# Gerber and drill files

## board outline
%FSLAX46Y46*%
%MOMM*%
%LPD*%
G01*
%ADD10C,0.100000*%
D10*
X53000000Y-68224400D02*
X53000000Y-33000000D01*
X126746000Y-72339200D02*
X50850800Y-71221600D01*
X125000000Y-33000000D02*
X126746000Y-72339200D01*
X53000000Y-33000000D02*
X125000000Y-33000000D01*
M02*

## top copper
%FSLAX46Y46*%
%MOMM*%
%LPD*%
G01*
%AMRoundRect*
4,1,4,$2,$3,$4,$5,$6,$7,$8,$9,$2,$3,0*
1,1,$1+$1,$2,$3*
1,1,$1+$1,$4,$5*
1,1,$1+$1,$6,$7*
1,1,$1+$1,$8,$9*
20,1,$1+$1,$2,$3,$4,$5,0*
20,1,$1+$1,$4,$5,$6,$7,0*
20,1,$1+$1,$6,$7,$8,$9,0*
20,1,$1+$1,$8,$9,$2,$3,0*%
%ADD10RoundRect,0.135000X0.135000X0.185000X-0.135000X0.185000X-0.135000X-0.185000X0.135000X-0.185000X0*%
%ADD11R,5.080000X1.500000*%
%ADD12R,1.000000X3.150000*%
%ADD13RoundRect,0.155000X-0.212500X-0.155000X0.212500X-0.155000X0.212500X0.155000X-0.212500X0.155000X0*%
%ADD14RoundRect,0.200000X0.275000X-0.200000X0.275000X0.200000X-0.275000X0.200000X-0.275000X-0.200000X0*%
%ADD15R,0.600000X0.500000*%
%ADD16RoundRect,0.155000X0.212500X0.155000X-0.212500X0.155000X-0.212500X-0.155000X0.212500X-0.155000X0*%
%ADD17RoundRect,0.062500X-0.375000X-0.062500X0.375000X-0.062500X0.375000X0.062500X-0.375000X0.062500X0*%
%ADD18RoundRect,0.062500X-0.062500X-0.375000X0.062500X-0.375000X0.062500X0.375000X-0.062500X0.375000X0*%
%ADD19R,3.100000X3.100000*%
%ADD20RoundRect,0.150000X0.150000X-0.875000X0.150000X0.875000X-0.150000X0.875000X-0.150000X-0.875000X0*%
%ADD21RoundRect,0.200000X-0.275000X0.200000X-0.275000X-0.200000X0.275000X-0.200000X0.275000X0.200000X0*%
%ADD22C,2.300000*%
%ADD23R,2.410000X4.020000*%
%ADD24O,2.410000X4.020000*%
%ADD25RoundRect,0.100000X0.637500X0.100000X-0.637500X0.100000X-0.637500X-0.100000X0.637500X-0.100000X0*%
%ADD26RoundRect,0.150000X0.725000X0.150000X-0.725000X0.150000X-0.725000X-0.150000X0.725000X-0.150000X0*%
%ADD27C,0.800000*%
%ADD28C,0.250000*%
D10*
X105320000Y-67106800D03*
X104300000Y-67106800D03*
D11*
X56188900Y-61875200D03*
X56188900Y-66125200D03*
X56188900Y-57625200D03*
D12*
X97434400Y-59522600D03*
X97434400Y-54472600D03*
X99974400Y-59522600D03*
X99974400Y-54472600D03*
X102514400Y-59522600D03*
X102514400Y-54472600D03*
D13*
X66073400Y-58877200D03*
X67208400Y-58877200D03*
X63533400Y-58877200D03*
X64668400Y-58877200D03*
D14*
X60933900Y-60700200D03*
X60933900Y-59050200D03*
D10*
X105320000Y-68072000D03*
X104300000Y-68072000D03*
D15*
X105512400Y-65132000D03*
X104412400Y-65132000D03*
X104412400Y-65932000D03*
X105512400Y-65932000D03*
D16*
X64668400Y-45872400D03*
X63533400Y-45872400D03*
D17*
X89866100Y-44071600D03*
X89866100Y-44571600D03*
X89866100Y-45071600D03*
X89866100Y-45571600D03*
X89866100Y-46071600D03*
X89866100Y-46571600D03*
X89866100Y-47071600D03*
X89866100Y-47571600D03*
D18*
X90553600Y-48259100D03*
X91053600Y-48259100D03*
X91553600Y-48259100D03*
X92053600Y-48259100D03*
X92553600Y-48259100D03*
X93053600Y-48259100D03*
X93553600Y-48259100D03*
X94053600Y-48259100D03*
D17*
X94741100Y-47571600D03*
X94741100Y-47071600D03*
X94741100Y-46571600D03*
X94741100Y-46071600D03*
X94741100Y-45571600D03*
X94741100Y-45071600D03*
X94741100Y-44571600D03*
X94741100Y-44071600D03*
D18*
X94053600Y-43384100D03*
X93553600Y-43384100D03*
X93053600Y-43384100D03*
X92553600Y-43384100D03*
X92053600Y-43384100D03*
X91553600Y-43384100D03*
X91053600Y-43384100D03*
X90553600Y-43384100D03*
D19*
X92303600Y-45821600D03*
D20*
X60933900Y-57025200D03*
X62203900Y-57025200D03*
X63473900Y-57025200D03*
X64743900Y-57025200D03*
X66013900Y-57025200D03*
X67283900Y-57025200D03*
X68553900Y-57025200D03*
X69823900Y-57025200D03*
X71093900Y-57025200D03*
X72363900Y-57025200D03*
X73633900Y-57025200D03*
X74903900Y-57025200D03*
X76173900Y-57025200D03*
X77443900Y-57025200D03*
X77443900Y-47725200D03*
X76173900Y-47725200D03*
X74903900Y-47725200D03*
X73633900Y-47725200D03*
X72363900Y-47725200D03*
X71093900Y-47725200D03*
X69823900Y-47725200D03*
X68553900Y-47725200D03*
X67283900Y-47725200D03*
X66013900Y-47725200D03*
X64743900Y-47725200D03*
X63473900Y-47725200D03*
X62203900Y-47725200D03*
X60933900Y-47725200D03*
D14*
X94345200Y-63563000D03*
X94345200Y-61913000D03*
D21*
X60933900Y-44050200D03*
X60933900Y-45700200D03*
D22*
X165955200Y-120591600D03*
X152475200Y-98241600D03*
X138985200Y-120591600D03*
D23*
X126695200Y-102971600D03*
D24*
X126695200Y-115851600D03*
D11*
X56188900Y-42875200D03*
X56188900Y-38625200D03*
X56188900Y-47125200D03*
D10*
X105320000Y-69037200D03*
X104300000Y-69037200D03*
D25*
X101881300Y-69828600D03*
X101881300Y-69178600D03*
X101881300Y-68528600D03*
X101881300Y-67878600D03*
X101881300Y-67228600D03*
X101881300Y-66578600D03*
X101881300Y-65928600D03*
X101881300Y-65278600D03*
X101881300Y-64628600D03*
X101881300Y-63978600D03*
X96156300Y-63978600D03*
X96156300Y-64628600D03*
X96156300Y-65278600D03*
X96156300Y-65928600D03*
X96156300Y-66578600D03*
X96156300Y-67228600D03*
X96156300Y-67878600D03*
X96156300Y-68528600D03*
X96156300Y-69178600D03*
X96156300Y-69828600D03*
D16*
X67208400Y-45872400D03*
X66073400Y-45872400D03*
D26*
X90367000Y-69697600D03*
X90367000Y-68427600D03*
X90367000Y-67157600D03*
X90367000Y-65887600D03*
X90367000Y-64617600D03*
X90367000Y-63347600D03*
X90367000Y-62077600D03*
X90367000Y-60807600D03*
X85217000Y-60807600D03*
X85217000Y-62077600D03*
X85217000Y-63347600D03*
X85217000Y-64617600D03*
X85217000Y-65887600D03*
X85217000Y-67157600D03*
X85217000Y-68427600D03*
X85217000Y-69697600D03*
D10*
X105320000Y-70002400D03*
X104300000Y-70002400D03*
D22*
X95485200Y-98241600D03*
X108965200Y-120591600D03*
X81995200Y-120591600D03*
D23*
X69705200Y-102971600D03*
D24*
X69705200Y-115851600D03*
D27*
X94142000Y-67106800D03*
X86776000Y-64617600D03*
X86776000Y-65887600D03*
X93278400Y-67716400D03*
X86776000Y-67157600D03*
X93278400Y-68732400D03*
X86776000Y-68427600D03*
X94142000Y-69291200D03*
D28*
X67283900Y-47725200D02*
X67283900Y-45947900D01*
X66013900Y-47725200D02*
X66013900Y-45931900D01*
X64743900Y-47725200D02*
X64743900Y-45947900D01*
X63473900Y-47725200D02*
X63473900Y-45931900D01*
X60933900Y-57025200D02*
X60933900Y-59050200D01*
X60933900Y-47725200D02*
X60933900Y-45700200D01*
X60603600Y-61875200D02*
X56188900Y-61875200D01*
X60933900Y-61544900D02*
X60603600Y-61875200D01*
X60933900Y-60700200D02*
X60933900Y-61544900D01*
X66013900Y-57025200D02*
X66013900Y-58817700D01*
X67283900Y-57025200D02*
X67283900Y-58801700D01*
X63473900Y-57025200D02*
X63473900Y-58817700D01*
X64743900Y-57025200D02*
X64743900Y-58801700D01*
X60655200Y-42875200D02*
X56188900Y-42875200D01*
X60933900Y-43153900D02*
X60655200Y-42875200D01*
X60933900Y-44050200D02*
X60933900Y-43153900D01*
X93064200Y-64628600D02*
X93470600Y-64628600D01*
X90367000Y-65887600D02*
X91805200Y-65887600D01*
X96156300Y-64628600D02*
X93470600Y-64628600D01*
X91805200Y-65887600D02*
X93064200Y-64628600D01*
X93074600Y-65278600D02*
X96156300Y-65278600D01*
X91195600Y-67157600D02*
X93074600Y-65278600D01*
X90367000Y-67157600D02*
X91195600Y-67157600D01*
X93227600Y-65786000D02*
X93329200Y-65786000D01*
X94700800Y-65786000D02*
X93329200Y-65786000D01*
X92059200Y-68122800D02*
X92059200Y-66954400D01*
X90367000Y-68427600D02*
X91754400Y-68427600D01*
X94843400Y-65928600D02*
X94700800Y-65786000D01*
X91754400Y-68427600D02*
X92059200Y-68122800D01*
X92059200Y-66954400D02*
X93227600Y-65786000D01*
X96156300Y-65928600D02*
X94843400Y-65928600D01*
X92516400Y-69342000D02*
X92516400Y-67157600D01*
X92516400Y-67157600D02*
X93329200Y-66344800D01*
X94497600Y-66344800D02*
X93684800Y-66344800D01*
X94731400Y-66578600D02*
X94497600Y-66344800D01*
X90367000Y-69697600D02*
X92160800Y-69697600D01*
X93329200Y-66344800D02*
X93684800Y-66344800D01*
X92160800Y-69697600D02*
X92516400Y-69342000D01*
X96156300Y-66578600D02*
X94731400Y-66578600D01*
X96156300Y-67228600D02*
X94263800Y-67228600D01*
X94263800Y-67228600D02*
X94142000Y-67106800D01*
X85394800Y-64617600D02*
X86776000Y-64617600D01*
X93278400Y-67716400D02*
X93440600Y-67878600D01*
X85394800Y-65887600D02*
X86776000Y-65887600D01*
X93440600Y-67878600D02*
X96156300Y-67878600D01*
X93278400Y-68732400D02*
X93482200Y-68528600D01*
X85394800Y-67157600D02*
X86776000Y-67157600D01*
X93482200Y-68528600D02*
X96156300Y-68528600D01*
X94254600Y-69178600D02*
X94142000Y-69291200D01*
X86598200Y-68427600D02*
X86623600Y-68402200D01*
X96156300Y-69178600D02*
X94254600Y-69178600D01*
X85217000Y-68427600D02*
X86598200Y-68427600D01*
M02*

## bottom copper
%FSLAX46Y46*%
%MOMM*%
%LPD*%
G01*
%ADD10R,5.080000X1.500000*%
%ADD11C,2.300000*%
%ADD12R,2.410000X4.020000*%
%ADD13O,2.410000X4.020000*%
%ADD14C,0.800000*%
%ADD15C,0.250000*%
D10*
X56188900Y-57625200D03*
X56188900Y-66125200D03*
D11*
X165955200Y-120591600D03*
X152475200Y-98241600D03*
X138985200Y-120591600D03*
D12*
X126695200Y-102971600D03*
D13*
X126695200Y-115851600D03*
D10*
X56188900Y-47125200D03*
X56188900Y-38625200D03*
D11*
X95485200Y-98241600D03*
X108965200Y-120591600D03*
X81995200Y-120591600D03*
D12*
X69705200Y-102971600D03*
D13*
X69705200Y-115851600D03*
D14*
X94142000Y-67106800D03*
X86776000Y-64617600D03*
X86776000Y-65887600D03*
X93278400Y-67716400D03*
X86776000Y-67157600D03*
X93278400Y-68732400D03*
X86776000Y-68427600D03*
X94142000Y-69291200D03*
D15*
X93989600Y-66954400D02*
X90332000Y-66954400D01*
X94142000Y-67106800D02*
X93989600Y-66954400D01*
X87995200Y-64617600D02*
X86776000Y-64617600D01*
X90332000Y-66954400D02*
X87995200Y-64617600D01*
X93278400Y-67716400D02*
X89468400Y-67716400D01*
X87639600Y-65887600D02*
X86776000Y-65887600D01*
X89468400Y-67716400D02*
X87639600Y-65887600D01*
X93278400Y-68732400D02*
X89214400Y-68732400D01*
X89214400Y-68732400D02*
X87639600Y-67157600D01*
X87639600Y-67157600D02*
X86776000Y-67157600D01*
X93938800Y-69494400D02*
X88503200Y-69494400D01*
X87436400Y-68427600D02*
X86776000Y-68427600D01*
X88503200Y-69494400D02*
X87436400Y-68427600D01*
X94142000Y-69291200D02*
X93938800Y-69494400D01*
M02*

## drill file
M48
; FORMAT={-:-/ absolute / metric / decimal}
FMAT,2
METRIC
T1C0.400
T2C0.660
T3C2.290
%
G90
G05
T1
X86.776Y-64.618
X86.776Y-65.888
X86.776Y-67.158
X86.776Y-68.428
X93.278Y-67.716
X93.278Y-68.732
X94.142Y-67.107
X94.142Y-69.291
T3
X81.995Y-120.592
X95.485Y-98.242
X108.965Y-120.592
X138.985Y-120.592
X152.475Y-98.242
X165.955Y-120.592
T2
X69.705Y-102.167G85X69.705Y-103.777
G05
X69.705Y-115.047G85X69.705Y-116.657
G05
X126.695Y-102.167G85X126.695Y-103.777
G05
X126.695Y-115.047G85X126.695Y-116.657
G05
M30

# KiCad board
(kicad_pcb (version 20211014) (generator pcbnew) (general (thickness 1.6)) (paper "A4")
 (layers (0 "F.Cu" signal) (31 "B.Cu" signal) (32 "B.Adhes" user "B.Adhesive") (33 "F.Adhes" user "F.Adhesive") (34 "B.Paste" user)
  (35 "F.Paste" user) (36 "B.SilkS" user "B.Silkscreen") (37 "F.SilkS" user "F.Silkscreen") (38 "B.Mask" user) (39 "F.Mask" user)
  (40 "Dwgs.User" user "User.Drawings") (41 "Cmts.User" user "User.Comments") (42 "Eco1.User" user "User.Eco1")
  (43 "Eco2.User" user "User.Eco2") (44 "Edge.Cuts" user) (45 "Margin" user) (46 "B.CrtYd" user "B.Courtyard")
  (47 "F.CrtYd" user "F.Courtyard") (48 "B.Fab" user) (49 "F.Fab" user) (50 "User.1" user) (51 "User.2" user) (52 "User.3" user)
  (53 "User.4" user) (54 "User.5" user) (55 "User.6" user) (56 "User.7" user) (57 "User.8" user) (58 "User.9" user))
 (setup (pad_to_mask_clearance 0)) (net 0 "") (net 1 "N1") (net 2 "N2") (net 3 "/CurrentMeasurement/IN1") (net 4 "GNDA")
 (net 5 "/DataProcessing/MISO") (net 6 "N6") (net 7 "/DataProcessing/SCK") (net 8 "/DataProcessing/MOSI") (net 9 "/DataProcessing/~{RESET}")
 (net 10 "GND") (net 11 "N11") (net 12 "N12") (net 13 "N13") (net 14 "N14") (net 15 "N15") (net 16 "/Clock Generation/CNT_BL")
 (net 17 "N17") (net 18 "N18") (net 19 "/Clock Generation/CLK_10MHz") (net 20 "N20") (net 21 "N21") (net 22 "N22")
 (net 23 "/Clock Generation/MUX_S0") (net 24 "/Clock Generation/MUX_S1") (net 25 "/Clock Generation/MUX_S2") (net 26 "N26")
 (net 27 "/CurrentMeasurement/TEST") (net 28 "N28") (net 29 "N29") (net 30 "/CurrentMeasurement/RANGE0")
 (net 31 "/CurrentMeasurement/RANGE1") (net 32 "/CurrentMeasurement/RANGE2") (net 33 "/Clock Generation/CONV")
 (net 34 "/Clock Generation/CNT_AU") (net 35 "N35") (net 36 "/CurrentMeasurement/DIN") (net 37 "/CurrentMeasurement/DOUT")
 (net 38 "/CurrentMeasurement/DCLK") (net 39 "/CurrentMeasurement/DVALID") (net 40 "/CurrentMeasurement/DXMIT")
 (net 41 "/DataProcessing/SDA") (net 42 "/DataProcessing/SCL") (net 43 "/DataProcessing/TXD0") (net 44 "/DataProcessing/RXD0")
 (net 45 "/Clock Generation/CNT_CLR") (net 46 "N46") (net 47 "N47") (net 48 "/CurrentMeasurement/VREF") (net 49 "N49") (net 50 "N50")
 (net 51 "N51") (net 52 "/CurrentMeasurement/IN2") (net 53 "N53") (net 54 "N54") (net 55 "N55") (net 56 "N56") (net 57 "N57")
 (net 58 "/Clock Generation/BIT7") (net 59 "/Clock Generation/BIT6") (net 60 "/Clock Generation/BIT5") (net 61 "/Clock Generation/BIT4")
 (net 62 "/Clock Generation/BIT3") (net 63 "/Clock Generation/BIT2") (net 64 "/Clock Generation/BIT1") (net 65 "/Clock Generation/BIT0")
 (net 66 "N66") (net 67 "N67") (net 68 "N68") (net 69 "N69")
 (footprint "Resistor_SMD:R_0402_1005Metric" (layer "F.Cu") (at 104.81 67.1068 180)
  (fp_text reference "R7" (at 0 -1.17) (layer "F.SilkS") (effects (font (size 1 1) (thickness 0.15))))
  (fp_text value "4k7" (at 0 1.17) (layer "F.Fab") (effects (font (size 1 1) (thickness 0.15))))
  (pad "1" smd roundrect (at -0.51 0 180) (size 0.54 0.64) (layers "F.Cu" "F.Paste" "F.Mask") (roundrect_rratio 0.25) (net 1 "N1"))
  (pad "2" smd roundrect (at 0.51 0 180) (size 0.54 0.64) (layers "F.Cu" "F.Paste" "F.Mask") (roundrect_rratio 0.25) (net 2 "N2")))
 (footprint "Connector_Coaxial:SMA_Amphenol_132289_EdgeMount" (layer "F.Cu") (at 56.1889 61.8752 180)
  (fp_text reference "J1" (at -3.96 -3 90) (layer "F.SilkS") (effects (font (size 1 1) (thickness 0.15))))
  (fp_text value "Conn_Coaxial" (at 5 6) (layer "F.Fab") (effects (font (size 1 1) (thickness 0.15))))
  (pad "1" smd rect (at 0 0 270) (size 1.5 5.08) (layers "F.Cu" "F.Paste" "F.Mask") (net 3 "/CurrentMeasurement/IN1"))
  (pad "2" smd rect (at 0 -4.25 270) (size 1.5 5.08) (layers "F.Cu" "F.Paste" "F.Mask") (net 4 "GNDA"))
  (pad "2" smd rect (at 0 4.25 270) (size 1.5 5.08) (layers "F.Cu" "F.Paste" "F.Mask") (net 4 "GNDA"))
  (pad "2" smd rect (at 0 4.25 270) (size 1.5 5.08) (layers "B.Cu" "B.Paste" "B.Mask") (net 4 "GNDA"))
  (pad "2" smd rect (at 0 -4.25 270) (size 1.5 5.08) (layers "B.Cu" "B.Paste" "B.Mask") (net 4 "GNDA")))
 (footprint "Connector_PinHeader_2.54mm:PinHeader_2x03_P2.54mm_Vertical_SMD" (layer "F.Cu") (at 99.9744 56.9976 90)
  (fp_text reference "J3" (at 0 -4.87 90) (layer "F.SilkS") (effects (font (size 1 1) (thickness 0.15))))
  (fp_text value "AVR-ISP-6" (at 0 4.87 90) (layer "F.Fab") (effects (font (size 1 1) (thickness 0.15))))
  (pad "1" smd rect (at -2.525 -2.54 90) (size 3.15 1) (layers "F.Cu" "F.Paste" "F.Mask") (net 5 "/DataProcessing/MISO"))
  (pad "2" smd rect (at 2.525 -2.54 90) (size 3.15 1) (layers "F.Cu" "F.Paste" "F.Mask") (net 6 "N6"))
  (pad "3" smd rect (at -2.525 0 90) (size 3.15 1) (layers "F.Cu" "F.Paste" "F.Mask") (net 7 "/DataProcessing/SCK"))
  (pad "4" smd rect (at 2.525 0 90) (size 3.15 1) (layers "F.Cu" "F.Paste" "F.Mask") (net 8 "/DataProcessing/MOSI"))
  (pad "5" smd rect (at -2.525 2.54 90) (size 3.15 1) (layers "F.Cu" "F.Paste" "F.Mask") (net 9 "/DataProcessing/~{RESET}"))
  (pad "6" smd rect (at 2.525 2.54 90) (size 3.15 1) (layers "F.Cu" "F.Paste" "F.Mask") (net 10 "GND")))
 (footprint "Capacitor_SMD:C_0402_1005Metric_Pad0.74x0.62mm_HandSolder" (layer "F.Cu") (at 66.6409 58.8772)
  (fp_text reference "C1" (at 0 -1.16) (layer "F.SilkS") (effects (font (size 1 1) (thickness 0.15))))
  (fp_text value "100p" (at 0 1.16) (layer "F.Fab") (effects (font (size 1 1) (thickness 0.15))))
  (pad "1" smd roundrect (at -0.5675 0) (size 0.735 0.62) (layers "F.Cu" "F.Paste" "F.Mask") (roundrect_rratio 0.25) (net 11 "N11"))
  (pad "2" smd roundrect (at 0.5675 0) (size 0.735 0.62) (layers "F.Cu" "F.Paste" "F.Mask") (roundrect_rratio 0.25) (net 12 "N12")))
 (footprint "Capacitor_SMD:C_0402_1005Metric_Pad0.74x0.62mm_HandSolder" (layer "F.Cu") (at 64.1009 58.8772)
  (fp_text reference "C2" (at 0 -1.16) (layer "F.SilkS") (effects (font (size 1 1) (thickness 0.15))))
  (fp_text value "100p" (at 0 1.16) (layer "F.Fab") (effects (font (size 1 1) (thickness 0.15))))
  (pad "1" smd roundrect (at -0.5675 0) (size 0.735 0.62) (layers "F.Cu" "F.Paste" "F.Mask") (roundrect_rratio 0.25) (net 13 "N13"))
  (pad "2" smd roundrect (at 0.5675 0) (size 0.735 0.62) (layers "F.Cu" "F.Paste" "F.Mask") (roundrect_rratio 0.25) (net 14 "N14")))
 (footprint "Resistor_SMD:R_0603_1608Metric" (layer "F.Cu") (at 60.9339 59.8752 90)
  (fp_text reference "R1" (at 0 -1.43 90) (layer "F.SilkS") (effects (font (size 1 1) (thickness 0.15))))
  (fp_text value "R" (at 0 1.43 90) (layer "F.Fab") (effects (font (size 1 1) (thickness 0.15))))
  (pad "1" smd roundrect (at -0.825 0 90) (size 0.8 0.95) (layers "F.Cu" "F.Paste" "F.Mask") (roundrect_rratio 0.25)
   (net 3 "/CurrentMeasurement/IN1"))
  (pad "2" smd roundrect (at 0.825 0 90) (size 0.8 0.95) (layers "F.Cu" "F.Paste" "F.Mask") (roundrect_rratio 0.25) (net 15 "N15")))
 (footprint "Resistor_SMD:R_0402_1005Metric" (layer "F.Cu") (at 104.81 68.072 180)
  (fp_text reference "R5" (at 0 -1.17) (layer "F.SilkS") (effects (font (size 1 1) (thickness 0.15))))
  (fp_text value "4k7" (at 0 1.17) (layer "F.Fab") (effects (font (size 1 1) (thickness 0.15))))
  (pad "1" smd roundrect (at -0.51 0 180) (size 0.54 0.64) (layers "F.Cu" "F.Paste" "F.Mask") (roundrect_rratio 0.25)
   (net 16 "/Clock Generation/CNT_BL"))
  (pad "2" smd roundrect (at 0.51 0 180) (size 0.54 0.64) (layers "F.Cu" "F.Paste" "F.Mask") (roundrect_rratio 0.25) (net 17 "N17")))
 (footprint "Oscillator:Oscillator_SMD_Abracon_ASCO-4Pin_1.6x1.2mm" (layer "F.Cu") (at 104.9624 65.532 -90)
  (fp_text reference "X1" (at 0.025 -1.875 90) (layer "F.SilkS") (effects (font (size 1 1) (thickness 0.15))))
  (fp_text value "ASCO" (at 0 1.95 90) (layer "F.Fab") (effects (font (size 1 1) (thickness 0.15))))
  (pad "1" smd rect (at -0.4 -0.55 270) (size 0.5 0.6) (layers "F.Cu" "F.Paste" "F.Mask") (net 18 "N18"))
  (pad "2" smd rect (at -0.4 0.55 270) (size 0.5 0.6) (layers "F.Cu" "F.Paste" "F.Mask") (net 10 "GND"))
  (pad "3" smd rect (at 0.4 0.55 270) (size 0.5 0.6) (layers "F.Cu" "F.Paste" "F.Mask") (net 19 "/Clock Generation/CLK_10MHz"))
  (pad "4" smd rect (at 0.4 -0.55 270) (size 0.5 0.6) (layers "F.Cu" "F.Paste" "F.Mask") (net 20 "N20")))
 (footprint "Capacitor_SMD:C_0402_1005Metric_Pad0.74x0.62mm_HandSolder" (layer "F.Cu") (at 64.1009 45.8724 180)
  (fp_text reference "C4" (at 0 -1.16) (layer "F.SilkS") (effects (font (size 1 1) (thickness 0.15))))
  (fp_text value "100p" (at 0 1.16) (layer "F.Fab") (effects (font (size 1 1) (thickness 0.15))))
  (pad "1" smd roundrect (at -0.5675 0 180) (size 0.735 0.62) (layers "F.Cu" "F.Paste" "F.Mask") (roundrect_rratio 0.25) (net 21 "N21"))
  (pad "2" smd roundrect (at 0.5675 0 180) (size 0.735 0.62) (layers "F.Cu" "F.Paste" "F.Mask") (roundrect_rratio 0.25) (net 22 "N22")))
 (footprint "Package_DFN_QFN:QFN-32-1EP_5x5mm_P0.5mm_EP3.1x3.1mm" (layer "F.Cu") (at 92.3036 45.8216)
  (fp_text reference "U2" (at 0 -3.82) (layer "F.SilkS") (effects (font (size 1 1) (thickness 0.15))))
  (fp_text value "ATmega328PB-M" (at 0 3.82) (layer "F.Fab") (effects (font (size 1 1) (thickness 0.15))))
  (pad "" smd roundrect (at -1.03 0) (size 0.83 0.83) (layers "F.Paste") (roundrect_rratio 0.25))
  (pad "" smd roundrect (at -1.03 1.03) (size 0.83 0.83) (layers "F.Paste") (roundrect_rratio 0.25))
  (pad "" smd roundrect (at 1.03 0) (size 0.83 0.83) (layers "F.Paste") (roundrect_rratio 0.25))
  (pad "" smd roundrect (at 1.03 1.03) (size 0.83 0.83) (layers "F.Paste") (roundrect_rratio 0.25))
  (pad "" smd roundrect (at 0 0) (size 0.83 0.83) (layers "F.Paste") (roundrect_rratio 0.25))
  (pad "" smd roundrect (at 1.03 -1.03) (size 0.83 0.83) (layers "F.Paste") (roundrect_rratio 0.25))
  (pad "" smd roundrect (at 0 -1.03) (size 0.83 0.83) (layers "F.Paste") (roundrect_rratio 0.25))
  (pad "" smd roundrect (at 0 1.03) (size 0.83 0.83) (layers "F.Paste") (roundrect_rratio 0.25))
  (pad "" smd roundrect (at -1.03 -1.03) (size 0.83 0.83) (layers "F.Paste") (roundrect_rratio 0.25))
  (pad "1" smd roundrect (at -2.4375 -1.75) (size 0.875 0.25) (layers "F.Cu" "F.Paste" "F.Mask") (roundrect_rratio 0.25)
   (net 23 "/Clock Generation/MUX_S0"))
  (pad "2" smd roundrect (at -2.4375 -1.25) (size 0.875 0.25) (layers "F.Cu" "F.Paste" "F.Mask") (roundrect_rratio 0.25)
   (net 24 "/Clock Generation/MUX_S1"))
  (pad "3" smd roundrect (at -2.4375 -0.75) (size 0.875 0.25) (layers "F.Cu" "F.Paste" "F.Mask") (roundrect_rratio 0.25)
   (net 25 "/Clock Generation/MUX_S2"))
  (pad "4" smd roundrect (at -2.4375 -0.25) (size 0.875 0.25) (layers "F.Cu" "F.Paste" "F.Mask") (roundrect_rratio 0.25) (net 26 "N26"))
  (pad "5" smd roundrect (at -2.4375 0.25) (size 0.875 0.25) (layers "F.Cu" "F.Paste" "F.Mask") (roundrect_rratio 0.25) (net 10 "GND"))
  (pad "6" smd roundrect (at -2.4375 0.75) (size 0.875 0.25) (layers "F.Cu" "F.Paste" "F.Mask") (roundrect_rratio 0.25)
   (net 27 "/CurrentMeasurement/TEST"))
  (pad "7" smd roundrect (at -2.4375 1.25) (size 0.875 0.25) (layers "F.Cu" "F.Paste" "F.Mask") (roundrect_rratio 0.25) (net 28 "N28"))
  (pad "8" smd roundrect (at -2.4375 1.75) (size 0.875 0.25) (layers "F.Cu" "F.Paste" "F.Mask") (roundrect_rratio 0.25) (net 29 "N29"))
  (pad "9" smd roundrect (at -1.75 2.4375) (size 0.25 0.875) (layers "F.Cu" "F.Paste" "F.Mask") (roundrect_rratio 0.25)
   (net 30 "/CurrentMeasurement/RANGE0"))
  (pad "10" smd roundrect (at -1.25 2.4375) (size 0.25 0.875) (layers "F.Cu" "F.Paste" "F.Mask") (roundrect_rratio 0.25)
   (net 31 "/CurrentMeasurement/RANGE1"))
  (pad "11" smd roundrect (at -0.75 2.4375) (size 0.25 0.875) (layers "F.Cu" "F.Paste" "F.Mask") (roundrect_rratio 0.25)
   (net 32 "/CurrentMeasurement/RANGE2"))
  (pad "12" smd roundrect (at -0.25 2.4375) (size 0.25 0.875) (layers "F.Cu" "F.Paste" "F.Mask") (roundrect_rratio 0.25)
   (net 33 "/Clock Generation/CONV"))
  (pad "13" smd roundrect (at 0.25 2.4375) (size 0.25 0.875) (layers "F.Cu" "F.Paste" "F.Mask") (roundrect_rratio 0.25)
   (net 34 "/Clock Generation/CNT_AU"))
  (pad "14" smd roundrect (at 0.75 2.4375) (size 0.25 0.875) (layers "F.Cu" "F.Paste" "F.Mask") (roundrect_rratio 0.25)
   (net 16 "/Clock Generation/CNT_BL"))
  (pad "15" smd roundrect (at 1.25 2.4375) (size 0.25 0.875) (layers "F.Cu" "F.Paste" "F.Mask") (roundrect_rratio 0.25)
   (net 8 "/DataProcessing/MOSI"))
  (pad "16" smd roundrect (at 1.75 2.4375) (size 0.25 0.875) (layers "F.Cu" "F.Paste" "F.Mask") (roundrect_rratio 0.25)
   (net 5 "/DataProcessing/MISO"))
  (pad "17" smd roundrect (at 2.4375 1.75) (size 0.875 0.25) (layers "F.Cu" "F.Paste" "F.Mask") (roundrect_rratio 0.25)
   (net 7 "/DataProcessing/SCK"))
  (pad "18" smd roundrect (at 2.4375 1.25) (size 0.875 0.25) (layers "F.Cu" "F.Paste" "F.Mask") (roundrect_rratio 0.25) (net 26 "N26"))
  (pad "19" smd roundrect (at 2.4375 0.75) (size 0.875 0.25) (layers "F.Cu" "F.Paste" "F.Mask") (roundrect_rratio 0.25) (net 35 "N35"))
  (pad "20" smd roundrect (at 2.4375 0.25) (size 0.875 0.25) (layers "F.Cu" "F.Paste" "F.Mask") (roundrect_rratio 0.25) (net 26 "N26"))
  (pad "21" smd roundrect (at 2.4375 -0.25) (size 0.875 0.25) (layers "F.Cu" "F.Paste" "F.Mask") (roundrect_rratio 0.25) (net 10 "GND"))
  (pad "22" smd roundrect (at 2.4375 -0.75) (size 0.875 0.25) (layers "F.Cu" "F.Paste" "F.Mask") (roundrect_rratio 0.25)
   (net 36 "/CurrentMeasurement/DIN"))
  (pad "23" smd roundrect (at 2.4375 -1.25) (size 0.875 0.25) (layers "F.Cu" "F.Paste" "F.Mask") (roundrect_rratio 0.25)
   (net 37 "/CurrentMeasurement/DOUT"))
  (pad "24" smd roundrect (at 2.4375 -1.75) (size 0.875 0.25) (layers "F.Cu" "F.Paste" "F.Mask") (roundrect_rratio 0.25)
   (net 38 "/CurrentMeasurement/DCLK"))
  (pad "25" smd roundrect (at 1.75 -2.4375) (size 0.25 0.875) (layers "F.Cu" "F.Paste" "F.Mask") (roundrect_rratio 0.25)
   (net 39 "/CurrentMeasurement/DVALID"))
  (pad "26" smd roundrect (at 1.25 -2.4375) (size 0.25 0.875) (layers "F.Cu" "F.Paste" "F.Mask") (roundrect_rratio 0.25)
   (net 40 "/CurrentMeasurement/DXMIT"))
  (pad "27" smd roundrect (at 0.75 -2.4375) (size 0.25 0.875) (layers "F.Cu" "F.Paste" "F.Mask") (roundrect_rratio 0.25)
   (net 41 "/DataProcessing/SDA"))
  (pad "28" smd roundrect (at 0.25 -2.4375) (size 0.25 0.875) (layers "F.Cu" "F.Paste" "F.Mask") (roundrect_rratio 0.25)
   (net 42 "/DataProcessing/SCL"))
  (pad "29" smd roundrect (at -0.25 -2.4375) (size 0.25 0.875) (layers "F.Cu" "F.Paste" "F.Mask") (roundrect_rratio 0.25)
   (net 9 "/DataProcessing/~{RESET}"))
  (pad "30" smd roundrect (at -0.75 -2.4375) (size 0.25 0.875) (layers "F.Cu" "F.Paste" "F.Mask") (roundrect_rratio 0.25)
   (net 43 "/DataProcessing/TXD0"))
  (pad "31" smd roundrect (at -1.25 -2.4375) (size 0.25 0.875) (layers "F.Cu" "F.Paste" "F.Mask") (roundrect_rratio 0.25)
   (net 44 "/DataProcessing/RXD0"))
  (pad "32" smd roundrect (at -1.75 -2.4375) (size 0.25 0.875) (layers "F.Cu" "F.Paste" "F.Mask") (roundrect_rratio 0.25)
   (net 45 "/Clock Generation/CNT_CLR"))
  (pad "33" smd rect (at 0 0) (size 3.1 3.1) (layers "F.Cu" "F.Mask") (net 10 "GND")))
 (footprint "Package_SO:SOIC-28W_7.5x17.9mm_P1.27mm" (layer "F.Cu") (at 69.1889 52.3752 90)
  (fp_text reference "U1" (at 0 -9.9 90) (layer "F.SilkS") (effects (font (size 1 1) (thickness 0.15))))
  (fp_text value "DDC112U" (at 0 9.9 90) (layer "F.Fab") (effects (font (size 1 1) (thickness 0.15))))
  (pad "1" smd roundrect (at -4.65 -8.255 90) (size 2.05 0.6) (layers "F.Cu" "F.Paste" "F.Mask") (roundrect_rratio 0.25) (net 15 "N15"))
  (pad "2" smd roundrect (at -4.65 -6.985 90) (size 2.05 0.6) (layers "F.Cu" "F.Paste" "F.Mask") (roundrect_rratio 0.25) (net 4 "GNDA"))
  (pad "3" smd roundrect (at -4.65 -5.715 90) (size 2.05 0.6) (layers "F.Cu" "F.Paste" "F.Mask") (roundrect_rratio 0.25) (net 13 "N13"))
  (pad "4" smd roundrect (at -4.65 -4.445 90) (size 2.05 0.6) (layers "F.Cu" "F.Paste" "F.Mask") (roundrect_rratio 0.25) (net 14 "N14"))
  (pad "5" smd roundrect (at -4.65 -3.175 90) (size 2.05 0.6) (layers "F.Cu" "F.Paste" "F.Mask") (roundrect_rratio 0.25) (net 11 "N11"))
  (pad "6" smd roundrect (at -4.65 -1.905 90) (size 2.05 0.6) (layers "F.Cu" "F.Paste" "F.Mask") (roundrect_rratio 0.25) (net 12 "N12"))
  (pad "7" smd roundrect (at -4.65 -0.635 90) (size 2.05 0.6) (layers "F.Cu" "F.Paste" "F.Mask") (roundrect_rratio 0.25) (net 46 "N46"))
  (pad "8" smd roundrect (at -4.65 0.635 90) (size 2.05 0.6) (layers "F.Cu" "F.Paste" "F.Mask") (roundrect_rratio 0.25)
   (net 27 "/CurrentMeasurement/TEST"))
  (pad "9" smd roundrect (at -4.65 1.905 90) (size 2.05 0.6) (layers "F.Cu" "F.Paste" "F.Mask") (roundrect_rratio 0.25)
   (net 33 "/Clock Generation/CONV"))
  (pad "10" smd roundrect (at -4.65 3.175 90) (size 2.05 0.6) (layers "F.Cu" "F.Paste" "F.Mask") (roundrect_rratio 0.25)
   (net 19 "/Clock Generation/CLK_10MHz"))
  (pad "11" smd roundrect (at -4.65 4.445 90) (size 2.05 0.6) (layers "F.Cu" "F.Paste" "F.Mask") (roundrect_rratio 0.25)
   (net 38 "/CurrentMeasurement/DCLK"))
  (pad "12" smd roundrect (at -4.65 5.715 90) (size 2.05 0.6) (layers "F.Cu" "F.Paste" "F.Mask") (roundrect_rratio 0.25)
   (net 40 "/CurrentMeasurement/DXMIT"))
  (pad "13" smd roundrect (at -4.65 6.985 90) (size 2.05 0.6) (layers "F.Cu" "F.Paste" "F.Mask") (roundrect_rratio 0.25)
   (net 36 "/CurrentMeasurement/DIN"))
  (pad "14" smd roundrect (at -4.65 8.255 90) (size 2.05 0.6) (layers "F.Cu" "F.Paste" "F.Mask") (roundrect_rratio 0.25) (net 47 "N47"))
  (pad "15" smd roundrect (at 4.65 8.255 90) (size 2.05 0.6) (layers "F.Cu" "F.Paste" "F.Mask") (roundrect_rratio 0.25) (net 10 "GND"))
  (pad "16" smd roundrect (at 4.65 6.985 90) (size 2.05 0.6) (layers "F.Cu" "F.Paste" "F.Mask") (roundrect_rratio 0.25)
   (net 37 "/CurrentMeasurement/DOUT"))
  (pad "17" smd roundrect (at 4.65 5.715 90) (size 2.05 0.6) (layers "F.Cu" "F.Paste" "F.Mask") (roundrect_rratio 0.25)
   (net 39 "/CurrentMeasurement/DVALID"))
  (pad "18" smd roundrect (at 4.65 4.445 90) (size 2.05 0.6) (layers "F.Cu" "F.Paste" "F.Mask") (roundrect_rratio 0.25)
   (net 30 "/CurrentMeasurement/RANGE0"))
  (pad "19" smd roundrect (at 4.65 3.175 90) (size 2.05 0.6) (layers "F.Cu" "F.Paste" "F.Mask") (roundrect_rratio 0.25)
   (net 31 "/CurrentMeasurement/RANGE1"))
  (pad "20" smd roundrect (at 4.65 1.905 90) (size 2.05 0.6) (layers "F.Cu" "F.Paste" "F.Mask") (roundrect_rratio 0.25)
   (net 32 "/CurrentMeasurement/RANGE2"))
  (pad "21" smd roundrect (at 4.65 0.635 90) (size 2.05 0.6) (layers "F.Cu" "F.Paste" "F.Mask") (roundrect_rratio 0.25) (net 4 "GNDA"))
  (pad "22" smd roundrect (at 4.65 -0.635 90) (size 2.05 0.6) (layers "F.Cu" "F.Paste" "F.Mask") (roundrect_rratio 0.25)
   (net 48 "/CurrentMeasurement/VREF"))
  (pad "23" smd roundrect (at 4.65 -1.905 90) (size 2.05 0.6) (layers "F.Cu" "F.Paste" "F.Mask") (roundrect_rratio 0.25) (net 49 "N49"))
  (pad "24" smd roundrect (at 4.65 -3.175 90) (size 2.05 0.6) (layers "F.Cu" "F.Paste" "F.Mask") (roundrect_rratio 0.25) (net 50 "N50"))
  (pad "25" smd roundrect (at 4.65 -4.445 90) (size 2.05 0.6) (layers "F.Cu" "F.Paste" "F.Mask") (roundrect_rratio 0.25) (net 21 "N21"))
  (pad "26" smd roundrect (at 4.65 -5.715 90) (size 2.05 0.6) (layers "F.Cu" "F.Paste" "F.Mask") (roundrect_rratio 0.25) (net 22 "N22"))
  (pad "27" smd roundrect (at 4.65 -6.985 90) (size 2.05 0.6) (layers "F.Cu" "F.Paste" "F.Mask") (roundrect_rratio 0.25) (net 4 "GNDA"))
  (pad "28" smd roundrect (at 4.65 -8.255 90) (size 2.05 0.6) (layers "F.Cu" "F.Paste" "F.Mask") (roundrect_rratio 0.25) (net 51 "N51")))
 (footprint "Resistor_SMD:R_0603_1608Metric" (layer "F.Cu") (at 94.3452 62.738 90)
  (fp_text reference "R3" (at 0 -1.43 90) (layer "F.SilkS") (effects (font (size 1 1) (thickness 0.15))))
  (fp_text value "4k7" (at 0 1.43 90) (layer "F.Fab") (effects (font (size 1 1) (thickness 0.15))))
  (pad "1" smd roundrect (at -0.825 0 90) (size 0.8 0.95) (layers "F.Cu" "F.Paste" "F.Mask") (roundrect_rratio 0.25)
   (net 45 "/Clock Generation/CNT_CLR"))
  (pad "2" smd roundrect (at 0.825 0 90) (size 0.8 0.95) (layers "F.Cu" "F.Paste" "F.Mask") (roundrect_rratio 0.25) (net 10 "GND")))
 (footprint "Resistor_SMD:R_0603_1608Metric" (layer "F.Cu") (at 60.9339 44.8752 -90)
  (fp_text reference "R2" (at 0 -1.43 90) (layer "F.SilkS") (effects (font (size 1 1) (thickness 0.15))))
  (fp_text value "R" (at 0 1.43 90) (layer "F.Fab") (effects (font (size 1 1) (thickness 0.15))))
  (pad "1" smd roundrect (at -0.825 0 270) (size 0.8 0.95) (layers "F.Cu" "F.Paste" "F.Mask") (roundrect_rratio 0.25)
   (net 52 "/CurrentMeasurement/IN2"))
  (pad "2" smd roundrect (at 0.825 0 270) (size 0.8 0.95) (layers "F.Cu" "F.Paste" "F.Mask") (roundrect_rratio 0.25) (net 51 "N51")))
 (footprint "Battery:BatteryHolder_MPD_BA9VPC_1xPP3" (layer "F.Cu") (at 126.6952 102.9716)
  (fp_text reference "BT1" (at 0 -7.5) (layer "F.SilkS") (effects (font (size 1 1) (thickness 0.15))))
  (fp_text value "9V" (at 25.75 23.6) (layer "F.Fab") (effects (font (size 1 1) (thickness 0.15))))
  (pad "" np_thru_hole circle (at 39.26 17.62) (size 2.3 2.3) (drill 2.29) (layers *.Cu *.Mask))
  (pad "" np_thru_hole circle (at 25.78 -4.73) (size 2.3 2.3) (drill 2.29) (layers *.Cu *.Mask))
  (pad "" np_thru_hole circle (at 12.29 17.62) (size 2.3 2.3) (drill 2.29) (layers *.Cu *.Mask))
  (pad "1" thru_hole rect (at 0 0) (size 2.41 4.02) (drill oval 0.66 2.27) (layers *.Cu *.Mask) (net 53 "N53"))
  (pad "2" thru_hole oval (at 0 12.88) (size 2.41 4.02) (drill oval 0.66 2.27) (layers *.Cu *.Mask) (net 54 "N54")))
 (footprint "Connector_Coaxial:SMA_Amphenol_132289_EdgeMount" (layer "F.Cu") (at 56.1889 42.8752 180)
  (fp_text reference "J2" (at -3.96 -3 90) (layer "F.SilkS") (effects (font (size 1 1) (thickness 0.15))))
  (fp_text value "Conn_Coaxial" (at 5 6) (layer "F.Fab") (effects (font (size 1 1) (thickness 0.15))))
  (pad "1" smd rect (at 0 0 270) (size 1.5 5.08) (layers "F.Cu" "F.Paste" "F.Mask") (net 52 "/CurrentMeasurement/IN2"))
  (pad "2" smd rect (at 0 -4.25 270) (size 1.5 5.08) (layers "B.Cu" "B.Paste" "B.Mask") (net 4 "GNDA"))
  (pad "2" smd rect (at 0 4.25 270) (size 1.5 5.08) (layers "F.Cu" "F.Paste" "F.Mask") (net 4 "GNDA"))
  (pad "2" smd rect (at 0 -4.25 270) (size 1.5 5.08) (layers "F.Cu" "F.Paste" "F.Mask") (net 4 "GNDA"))
  (pad "2" smd rect (at 0 4.25 270) (size 1.5 5.08) (layers "B.Cu" "B.Paste" "B.Mask") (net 4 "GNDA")))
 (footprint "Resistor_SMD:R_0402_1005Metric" (layer "F.Cu") (at 104.81 69.0372 180)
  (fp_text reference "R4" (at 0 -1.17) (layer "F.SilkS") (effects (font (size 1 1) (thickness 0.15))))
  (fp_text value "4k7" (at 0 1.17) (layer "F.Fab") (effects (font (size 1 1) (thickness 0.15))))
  (pad "1" smd roundrect (at -0.51 0 180) (size 0.54 0.64) (layers "F.Cu" "F.Paste" "F.Mask") (roundrect_rratio 0.25)
   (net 34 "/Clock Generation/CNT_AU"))
  (pad "2" smd roundrect (at 0.51 0 180) (size 0.54 0.64) (layers "F.Cu" "F.Paste" "F.Mask") (roundrect_rratio 0.25) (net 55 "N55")))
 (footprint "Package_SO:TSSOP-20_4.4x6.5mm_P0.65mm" (layer "F.Cu") (at 99.0188 66.9036 180)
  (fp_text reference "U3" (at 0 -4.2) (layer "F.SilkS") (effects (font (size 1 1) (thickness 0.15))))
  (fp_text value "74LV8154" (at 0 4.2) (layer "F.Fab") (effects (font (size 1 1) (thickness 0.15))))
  (pad "1" smd roundrect (at -2.8625 -2.925 180) (size 1.475 0.4) (layers "F.Cu" "F.Paste" "F.Mask") (roundrect_rratio 0.25)
   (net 19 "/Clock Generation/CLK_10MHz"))
  (pad "2" smd roundrect (at -2.8625 -2.275 180) (size 1.475 0.4) (layers "F.Cu" "F.Paste" "F.Mask") (roundrect_rratio 0.25)
   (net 19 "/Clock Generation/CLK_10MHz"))
  (pad "3" smd roundrect (at -2.8625 -1.625 180) (size 1.475 0.4) (layers "F.Cu" "F.Paste" "F.Mask") (roundrect_rratio 0.25) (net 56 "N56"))
  (pad "4" smd roundrect (at -2.8625 -0.975 180) (size 1.475 0.4) (layers "F.Cu" "F.Paste" "F.Mask") (roundrect_rratio 0.25) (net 55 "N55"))
  (pad "5" smd roundrect (at -2.8625 -0.325 180) (size 1.475 0.4) (layers "F.Cu" "F.Paste" "F.Mask") (roundrect_rratio 0.25) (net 17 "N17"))
  (pad "6" smd roundrect (at -2.8625 0.325 180) (size 1.475 0.4) (layers "F.Cu" "F.Paste" "F.Mask") (roundrect_rratio 0.25) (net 2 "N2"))
  (pad "7" smd roundrect (at -2.8625 0.975 180) (size 1.475 0.4) (layers "F.Cu" "F.Paste" "F.Mask") (roundrect_rratio 0.25)
   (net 19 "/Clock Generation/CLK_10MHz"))
  (pad "8" smd roundrect (at -2.8625 1.625 180) (size 1.475 0.4) (layers "F.Cu" "F.Paste" "F.Mask") (roundrect_rratio 0.25) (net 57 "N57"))
  (pad "9" smd roundrect (at -2.8625 2.275 180) (size 1.475 0.4) (layers "F.Cu" "F.Paste" "F.Mask") (roundrect_rratio 0.25) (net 57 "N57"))
  (pad "10" smd roundrect (at -2.8625 2.925 180) (size 1.475 0.4) (layers "F.Cu" "F.Paste" "F.Mask") (roundrect_rratio 0.25) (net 10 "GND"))
  (pad "11" smd roundrect (at 2.8625 2.925 180) (size 1.475 0.4) (layers "F.Cu" "F.Paste" "F.Mask") (roundrect_rratio 0.25)
   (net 45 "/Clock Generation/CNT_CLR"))
  (pad "12" smd roundrect (at 2.8625 2.275 180) (size 1.475 0.4) (layers "F.Cu" "F.Paste" "F.Mask") (roundrect_rratio 0.25)
   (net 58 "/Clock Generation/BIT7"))
  (pad "13" smd roundrect (at 2.8625 1.625 180) (size 1.475 0.4) (layers "F.Cu" "F.Paste" "F.Mask") (roundrect_rratio 0.25)
   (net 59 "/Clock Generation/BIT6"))
  (pad "14" smd roundrect (at 2.8625 0.975 180) (size 1.475 0.4) (layers "F.Cu" "F.Paste" "F.Mask") (roundrect_rratio 0.25)
   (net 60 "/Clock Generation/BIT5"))
  (pad "15" smd roundrect (at 2.8625 0.325 180) (size 1.475 0.4) (layers "F.Cu" "F.Paste" "F.Mask") (roundrect_rratio 0.25)
   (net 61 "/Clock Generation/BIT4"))
  (pad "16" smd roundrect (at 2.8625 -0.325 180) (size 1.475 0.4) (layers "F.Cu" "F.Paste" "F.Mask") (roundrect_rratio 0.25)
   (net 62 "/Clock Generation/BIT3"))
  (pad "17" smd roundrect (at 2.8625 -0.975 180) (size 1.475 0.4) (layers "F.Cu" "F.Paste" "F.Mask") (roundrect_rratio 0.25)
   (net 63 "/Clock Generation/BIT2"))
  (pad "18" smd roundrect (at 2.8625 -1.625 180) (size 1.475 0.4) (layers "F.Cu" "F.Paste" "F.Mask") (roundrect_rratio 0.25)
   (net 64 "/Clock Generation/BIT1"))
  (pad "19" smd roundrect (at 2.8625 -2.275 180) (size 1.475 0.4) (layers "F.Cu" "F.Paste" "F.Mask") (roundrect_rratio 0.25)
   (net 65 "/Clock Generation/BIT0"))
  (pad "20" smd roundrect (at 2.8625 -2.925 180) (size 1.475 0.4) (layers "F.Cu" "F.Paste" "F.Mask") (roundrect_rratio 0.25) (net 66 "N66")))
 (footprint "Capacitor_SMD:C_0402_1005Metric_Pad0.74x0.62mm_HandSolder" (layer "F.Cu") (at 66.6409 45.8724 180)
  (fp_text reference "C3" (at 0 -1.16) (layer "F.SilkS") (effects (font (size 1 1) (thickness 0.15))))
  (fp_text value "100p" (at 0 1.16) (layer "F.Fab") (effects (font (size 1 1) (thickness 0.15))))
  (pad "1" smd roundrect (at -0.5675 0 180) (size 0.735 0.62) (layers "F.Cu" "F.Paste" "F.Mask") (roundrect_rratio 0.25) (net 49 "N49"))
  (pad "2" smd roundrect (at 0.5675 0 180) (size 0.735 0.62) (layers "F.Cu" "F.Paste" "F.Mask") (roundrect_rratio 0.25) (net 50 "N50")))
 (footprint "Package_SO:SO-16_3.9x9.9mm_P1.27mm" (layer "F.Cu") (at 87.792 65.2526 180)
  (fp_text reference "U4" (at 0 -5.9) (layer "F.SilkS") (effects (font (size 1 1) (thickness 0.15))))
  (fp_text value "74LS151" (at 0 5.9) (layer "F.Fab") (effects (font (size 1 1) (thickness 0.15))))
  (pad "1" smd roundrect (at -2.575 -4.445 180) (size 1.75 0.6) (layers "F.Cu" "F.Paste" "F.Mask") (roundrect_rratio 0.25)
   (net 61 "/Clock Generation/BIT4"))
  (pad "2" smd roundrect (at -2.575 -3.175 180) (size 1.75 0.6) (layers "F.Cu" "F.Paste" "F.Mask") (roundrect_rratio 0.25)
   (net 60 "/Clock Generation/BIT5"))
  (pad "3" smd roundrect (at -2.575 -1.905 180) (size 1.75 0.6) (layers "F.Cu" "F.Paste" "F.Mask") (roundrect_rratio 0.25)
   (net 59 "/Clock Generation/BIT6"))
  (pad "4" smd roundrect (at -2.575 -0.635 180) (size 1.75 0.6) (layers "F.Cu" "F.Paste" "F.Mask") (roundrect_rratio 0.25)
   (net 58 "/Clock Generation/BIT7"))
  (pad "5" smd roundrect (at -2.575 0.635 180) (size 1.75 0.6) (layers "F.Cu" "F.Paste" "F.Mask") (roundrect_rratio 0.25)
   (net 33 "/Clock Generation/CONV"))
  (pad "6" smd roundrect (at -2.575 1.905 180) (size 1.75 0.6) (layers "F.Cu" "F.Paste" "F.Mask") (roundrect_rratio 0.25) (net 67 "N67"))
  (pad "7" smd roundrect (at -2.575 3.175 180) (size 1.75 0.6) (layers "F.Cu" "F.Paste" "F.Mask") (roundrect_rratio 0.25) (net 10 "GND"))
  (pad "8" smd roundrect (at -2.575 4.445 180) (size 1.75 0.6) (layers "F.Cu" "F.Paste" "F.Mask") (roundrect_rratio 0.25) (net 10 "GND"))
  (pad "9" smd roundrect (at 2.575 4.445 180) (size 1.75 0.6) (layers "F.Cu" "F.Paste" "F.Mask") (roundrect_rratio 0.25)
   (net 25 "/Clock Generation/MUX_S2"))
  (pad "10" smd roundrect (at 2.575 3.175 180) (size 1.75 0.6) (layers "F.Cu" "F.Paste" "F.Mask") (roundrect_rratio 0.25)
   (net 24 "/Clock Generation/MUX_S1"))
  (pad "11" smd roundrect (at 2.575 1.905 180) (size 1.75 0.6) (layers "F.Cu" "F.Paste" "F.Mask") (roundrect_rratio 0.25)
   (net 23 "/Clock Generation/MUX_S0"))
  (pad "12" smd roundrect (at 2.575 0.635 180) (size 1.75 0.6) (layers "F.Cu" "F.Paste" "F.Mask") (roundrect_rratio 0.25)
   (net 62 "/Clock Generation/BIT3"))
  (pad "13" smd roundrect (at 2.575 -0.635 180) (size 1.75 0.6) (layers "F.Cu" "F.Paste" "F.Mask") (roundrect_rratio 0.25)
   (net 63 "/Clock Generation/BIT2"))
  (pad "14" smd roundrect (at 2.575 -1.905 180) (size 1.75 0.6) (layers "F.Cu" "F.Paste" "F.Mask") (roundrect_rratio 0.25)
   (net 64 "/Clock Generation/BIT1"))
  (pad "15" smd roundrect (at 2.575 -3.175 180) (size 1.75 0.6) (layers "F.Cu" "F.Paste" "F.Mask") (roundrect_rratio 0.25)
   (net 65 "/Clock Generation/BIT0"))
  (pad "16" smd roundrect (at 2.575 -4.445 180) (size 1.75 0.6) (layers "F.Cu" "F.Paste" "F.Mask") (roundrect_rratio 0.25) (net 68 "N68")))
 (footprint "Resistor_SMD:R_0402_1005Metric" (layer "F.Cu") (at 104.81 70.0024 180)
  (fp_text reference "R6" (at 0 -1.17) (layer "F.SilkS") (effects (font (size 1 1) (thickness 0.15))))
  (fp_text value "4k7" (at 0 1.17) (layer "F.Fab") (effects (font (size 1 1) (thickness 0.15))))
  (pad "1" smd roundrect (at -0.51 0 180) (size 0.54 0.64) (layers "F.Cu" "F.Paste" "F.Mask") (roundrect_rratio 0.25) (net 1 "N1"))
  (pad "2" smd roundrect (at 0.51 0 180) (size 0.54 0.64) (layers "F.Cu" "F.Paste" "F.Mask") (roundrect_rratio 0.25) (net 56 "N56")))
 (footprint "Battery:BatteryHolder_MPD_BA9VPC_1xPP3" (layer "F.Cu") (at 69.7052 102.9716)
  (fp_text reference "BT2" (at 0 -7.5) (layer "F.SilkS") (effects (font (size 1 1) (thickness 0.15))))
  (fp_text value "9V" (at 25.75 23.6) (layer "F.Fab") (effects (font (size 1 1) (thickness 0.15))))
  (pad "" np_thru_hole circle (at 25.78 -4.73) (size 2.3 2.3) (drill 2.29) (layers *.Cu *.Mask))
  (pad "" np_thru_hole circle (at 39.26 17.62) (size 2.3 2.3) (drill 2.29) (layers *.Cu *.Mask))
  (pad "" np_thru_hole circle (at 12.29 17.62) (size 2.3 2.3) (drill 2.29) (layers *.Cu *.Mask))
  (pad "1" thru_hole rect (at 0 0) (size 2.41 4.02) (drill oval 0.66 2.27) (layers *.Cu *.Mask) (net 54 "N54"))
  (pad "2" thru_hole oval (at 0 12.88) (size 2.41 4.02) (drill oval 0.66 2.27) (layers *.Cu *.Mask) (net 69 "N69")))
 (gr_line (start 53 68.2244) (end 53 33) (layer "Edge.Cuts") (width 0.1))
 (gr_line (start 126.746 72.3392) (end 50.8508 71.2216) (layer "Edge.Cuts") (width 0.1))
 (gr_line (start 125 33) (end 126.746 72.3392) (layer "Edge.Cuts") (width 0.1))
 (gr_line (start 53 33) (end 125 33) (layer "Edge.Cuts") (width 0.1))
 (segment (start 67.2839 47.7252) (end 67.2839 45.9479) (width 0.25) (layer "F.Cu") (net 49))
 (segment (start 66.0139 47.7252) (end 66.0139 45.9319) (width 0.25) (layer "F.Cu") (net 50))
 (segment (start 64.7439 47.7252) (end 64.7439 45.9479) (width 0.25) (layer "F.Cu") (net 21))
 (segment (start 63.4739 47.7252) (end 63.4739 45.9319) (width 0.25) (layer "F.Cu") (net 22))
 (segment (start 60.9339 57.0252) (end 60.9339 59.0502) (width 0.25) (layer "F.Cu") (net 15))
 (segment (start 60.9339 47.7252) (end 60.9339 45.7002) (width 0.25) (layer "F.Cu") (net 51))
 (segment (start 60.6036 61.8752) (end 56.1889 61.8752) (width 0.25) (layer "F.Cu") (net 3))
 (segment (start 60.9339 61.5449) (end 60.6036 61.8752) (width 0.25) (layer "F.Cu") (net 3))
 (segment (start 60.9339 60.7002) (end 60.9339 61.5449) (width 0.25) (layer "F.Cu") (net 3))
 (segment (start 66.0139 57.0252) (end 66.0139 58.8177) (width 0.25) (layer "F.Cu") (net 11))
 (segment (start 67.2839 57.0252) (end 67.2839 58.8017) (width 0.25) (layer "F.Cu") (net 12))
 (segment (start 63.4739 57.0252) (end 63.4739 58.8177) (width 0.25) (layer "F.Cu") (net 13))
 (segment (start 64.7439 57.0252) (end 64.7439 58.8017) (width 0.25) (layer "F.Cu") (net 14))
 (segment (start 60.6552 42.8752) (end 56.1889 42.8752) (width 0.25) (layer "F.Cu") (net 52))
 (segment (start 60.9339 43.1539) (end 60.6552 42.8752) (width 0.25) (layer "F.Cu") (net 52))
 (segment (start 60.9339 44.0502) (end 60.9339 43.1539) (width 0.25) (layer "F.Cu") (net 52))
 (segment (start 93.0642 64.6286) (end 93.4706 64.6286) (width 0.25) (layer "F.Cu") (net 58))
 (segment (start 90.367 65.8876) (end 91.8052 65.8876) (width 0.25) (layer "F.Cu") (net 58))
 (segment (start 96.1563 64.6286) (end 93.4706 64.6286) (width 0.25) (layer "F.Cu") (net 58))
 (segment (start 91.8052 65.8876) (end 93.0642 64.6286) (width 0.25) (layer "F.Cu") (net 58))
 (segment (start 93.0746 65.2786) (end 96.1563 65.2786) (width 0.25) (layer "F.Cu") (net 59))
 (segment (start 91.1956 67.1576) (end 93.0746 65.2786) (width 0.25) (layer "F.Cu") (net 59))
 (segment (start 90.367 67.1576) (end 91.1956 67.1576) (width 0.25) (layer "F.Cu") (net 59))
 (segment (start 93.2276 65.786) (end 93.3292 65.786) (width 0.25) (layer "F.Cu") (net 60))
 (segment (start 94.7008 65.786) (end 93.3292 65.786) (width 0.25) (layer "F.Cu") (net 60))
 (segment (start 92.0592 68.1228) (end 92.0592 66.9544) (width 0.25) (layer "F.Cu") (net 60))
 (segment (start 90.367 68.4276) (end 91.7544 68.4276) (width 0.25) (layer "F.Cu") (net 60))
 (segment (start 94.8434 65.9286) (end 94.7008 65.786) (width 0.25) (layer "F.Cu") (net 60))
 (segment (start 91.7544 68.4276) (end 92.0592 68.1228) (width 0.25) (layer "F.Cu") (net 60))
 (segment (start 92.0592 66.9544) (end 93.2276 65.786) (width 0.25) (layer "F.Cu") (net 60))
 (segment (start 96.1563 65.9286) (end 94.8434 65.9286) (width 0.25) (layer "F.Cu") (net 60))
 (segment (start 92.5164 69.342) (end 92.5164 67.1576) (width 0.25) (layer "F.Cu") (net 61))
 (segment (start 92.5164 67.1576) (end 93.3292 66.3448) (width 0.25) (layer "F.Cu") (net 61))
 (segment (start 94.4976 66.3448) (end 93.6848 66.3448) (width 0.25) (layer "F.Cu") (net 61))
 (segment (start 94.7314 66.5786) (end 94.4976 66.3448) (width 0.25) (layer "F.Cu") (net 61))
 (segment (start 90.367 69.6976) (end 92.1608 69.6976) (width 0.25) (layer "F.Cu") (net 61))
 (segment (start 93.3292 66.3448) (end 93.6848 66.3448) (width 0.25) (layer "F.Cu") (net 61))
 (segment (start 92.1608 69.6976) (end 92.5164 69.342) (width 0.25) (layer "F.Cu") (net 61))
 (segment (start 96.1563 66.5786) (end 94.7314 66.5786) (width 0.25) (layer "F.Cu") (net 61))
 (segment (start 96.1563 67.2286) (end 94.2638 67.2286) (width 0.25) (layer "F.Cu") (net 62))
 (segment (start 94.2638 67.2286) (end 94.142 67.1068) (width 0.25) (layer "F.Cu") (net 62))
 (segment (start 85.3948 64.6176) (end 86.776 64.6176) (width 0.25) (layer "F.Cu") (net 62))
 (via (at 94.142 67.1068) (size 0.8) (drill 0.4) (layers "F.Cu" "B.Cu") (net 62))
 (via (at 86.776 64.6176) (size 0.8) (drill 0.4) (layers "F.Cu" "B.Cu") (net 62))
 (segment (start 93.9896 66.9544) (end 90.332 66.9544) (width 0.25) (layer "B.Cu") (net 62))
 (segment (start 94.142 67.1068) (end 93.9896 66.9544) (width 0.25) (layer "B.Cu") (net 62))
 (segment (start 87.9952 64.6176) (end 86.776 64.6176) (width 0.25) (layer "B.Cu") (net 62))
 (segment (start 90.332 66.9544) (end 87.9952 64.6176) (width 0.25) (layer "B.Cu") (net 62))
 (segment (start 93.2784 67.7164) (end 93.4406 67.8786) (width 0.25) (layer "F.Cu") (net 63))
 (segment (start 85.3948 65.8876) (end 86.776 65.8876) (width 0.25) (layer "F.Cu") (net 63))
 (segment (start 93.4406 67.8786) (end 96.1563 67.8786) (width 0.25) (layer "F.Cu") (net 63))
 (via (at 86.776 65.8876) (size 0.8) (drill 0.4) (layers "F.Cu" "B.Cu") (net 63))
 (via (at 93.2784 67.7164) (size 0.8) (drill 0.4) (layers "F.Cu" "B.Cu") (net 63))
 (segment (start 93.2784 67.7164) (end 89.4684 67.7164) (width 0.25) (layer "B.Cu") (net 63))
 (segment (start 87.6396 65.8876) (end 86.776 65.8876) (width 0.25) (layer "B.Cu") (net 63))
 (segment (start 89.4684 67.7164) (end 87.6396 65.8876) (width 0.25) (layer "B.Cu") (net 63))
 (segment (start 93.2784 68.7324) (end 93.4822 68.5286) (width 0.25) (layer "F.Cu") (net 64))
 (segment (start 85.3948 67.1576) (end 86.776 67.1576) (width 0.25) (layer "F.Cu") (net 64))
 (segment (start 93.4822 68.5286) (end 96.1563 68.5286) (width 0.25) (layer "F.Cu") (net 64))
 (via (at 86.776 67.1576) (size 0.8) (drill 0.4) (layers "F.Cu" "B.Cu") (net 64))
 (via (at 93.2784 68.7324) (size 0.8) (drill 0.4) (layers "F.Cu" "B.Cu") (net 64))
 (segment (start 93.2784 68.7324) (end 89.2144 68.7324) (width 0.25) (layer "B.Cu") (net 64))
 (segment (start 89.2144 68.7324) (end 87.6396 67.1576) (width 0.25) (layer "B.Cu") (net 64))
 (segment (start 87.6396 67.1576) (end 86.776 67.1576) (width 0.25) (layer "B.Cu") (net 64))
 (segment (start 94.2546 69.1786) (end 94.142 69.2912) (width 0.25) (layer "F.Cu") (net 65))
 (segment (start 86.5982 68.4276) (end 86.6236 68.4022) (width 0.25) (layer "F.Cu") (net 65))
 (segment (start 96.1563 69.1786) (end 94.2546 69.1786) (width 0.25) (layer "F.Cu") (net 65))
 (segment (start 85.217 68.4276) (end 86.5982 68.4276) (width 0.25) (layer "F.Cu") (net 65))
 (via (at 86.776 68.4276) (size 0.8) (drill 0.4) (layers "F.Cu" "B.Cu") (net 65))
 (via (at 94.142 69.2912) (size 0.8) (drill 0.4) (layers "F.Cu" "B.Cu") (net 65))
 (segment (start 93.9388 69.4944) (end 88.5032 69.4944) (width 0.25) (layer "B.Cu") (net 65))
 (segment (start 87.4364 68.4276) (end 86.776 68.4276) (width 0.25) (layer "B.Cu") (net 65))
 (segment (start 88.5032 69.4944) (end 87.4364 68.4276) (width 0.25) (layer "B.Cu") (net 65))
 (segment (start 94.142 69.2912) (end 93.9388 69.4944) (width 0.25) (layer "B.Cu") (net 65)))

